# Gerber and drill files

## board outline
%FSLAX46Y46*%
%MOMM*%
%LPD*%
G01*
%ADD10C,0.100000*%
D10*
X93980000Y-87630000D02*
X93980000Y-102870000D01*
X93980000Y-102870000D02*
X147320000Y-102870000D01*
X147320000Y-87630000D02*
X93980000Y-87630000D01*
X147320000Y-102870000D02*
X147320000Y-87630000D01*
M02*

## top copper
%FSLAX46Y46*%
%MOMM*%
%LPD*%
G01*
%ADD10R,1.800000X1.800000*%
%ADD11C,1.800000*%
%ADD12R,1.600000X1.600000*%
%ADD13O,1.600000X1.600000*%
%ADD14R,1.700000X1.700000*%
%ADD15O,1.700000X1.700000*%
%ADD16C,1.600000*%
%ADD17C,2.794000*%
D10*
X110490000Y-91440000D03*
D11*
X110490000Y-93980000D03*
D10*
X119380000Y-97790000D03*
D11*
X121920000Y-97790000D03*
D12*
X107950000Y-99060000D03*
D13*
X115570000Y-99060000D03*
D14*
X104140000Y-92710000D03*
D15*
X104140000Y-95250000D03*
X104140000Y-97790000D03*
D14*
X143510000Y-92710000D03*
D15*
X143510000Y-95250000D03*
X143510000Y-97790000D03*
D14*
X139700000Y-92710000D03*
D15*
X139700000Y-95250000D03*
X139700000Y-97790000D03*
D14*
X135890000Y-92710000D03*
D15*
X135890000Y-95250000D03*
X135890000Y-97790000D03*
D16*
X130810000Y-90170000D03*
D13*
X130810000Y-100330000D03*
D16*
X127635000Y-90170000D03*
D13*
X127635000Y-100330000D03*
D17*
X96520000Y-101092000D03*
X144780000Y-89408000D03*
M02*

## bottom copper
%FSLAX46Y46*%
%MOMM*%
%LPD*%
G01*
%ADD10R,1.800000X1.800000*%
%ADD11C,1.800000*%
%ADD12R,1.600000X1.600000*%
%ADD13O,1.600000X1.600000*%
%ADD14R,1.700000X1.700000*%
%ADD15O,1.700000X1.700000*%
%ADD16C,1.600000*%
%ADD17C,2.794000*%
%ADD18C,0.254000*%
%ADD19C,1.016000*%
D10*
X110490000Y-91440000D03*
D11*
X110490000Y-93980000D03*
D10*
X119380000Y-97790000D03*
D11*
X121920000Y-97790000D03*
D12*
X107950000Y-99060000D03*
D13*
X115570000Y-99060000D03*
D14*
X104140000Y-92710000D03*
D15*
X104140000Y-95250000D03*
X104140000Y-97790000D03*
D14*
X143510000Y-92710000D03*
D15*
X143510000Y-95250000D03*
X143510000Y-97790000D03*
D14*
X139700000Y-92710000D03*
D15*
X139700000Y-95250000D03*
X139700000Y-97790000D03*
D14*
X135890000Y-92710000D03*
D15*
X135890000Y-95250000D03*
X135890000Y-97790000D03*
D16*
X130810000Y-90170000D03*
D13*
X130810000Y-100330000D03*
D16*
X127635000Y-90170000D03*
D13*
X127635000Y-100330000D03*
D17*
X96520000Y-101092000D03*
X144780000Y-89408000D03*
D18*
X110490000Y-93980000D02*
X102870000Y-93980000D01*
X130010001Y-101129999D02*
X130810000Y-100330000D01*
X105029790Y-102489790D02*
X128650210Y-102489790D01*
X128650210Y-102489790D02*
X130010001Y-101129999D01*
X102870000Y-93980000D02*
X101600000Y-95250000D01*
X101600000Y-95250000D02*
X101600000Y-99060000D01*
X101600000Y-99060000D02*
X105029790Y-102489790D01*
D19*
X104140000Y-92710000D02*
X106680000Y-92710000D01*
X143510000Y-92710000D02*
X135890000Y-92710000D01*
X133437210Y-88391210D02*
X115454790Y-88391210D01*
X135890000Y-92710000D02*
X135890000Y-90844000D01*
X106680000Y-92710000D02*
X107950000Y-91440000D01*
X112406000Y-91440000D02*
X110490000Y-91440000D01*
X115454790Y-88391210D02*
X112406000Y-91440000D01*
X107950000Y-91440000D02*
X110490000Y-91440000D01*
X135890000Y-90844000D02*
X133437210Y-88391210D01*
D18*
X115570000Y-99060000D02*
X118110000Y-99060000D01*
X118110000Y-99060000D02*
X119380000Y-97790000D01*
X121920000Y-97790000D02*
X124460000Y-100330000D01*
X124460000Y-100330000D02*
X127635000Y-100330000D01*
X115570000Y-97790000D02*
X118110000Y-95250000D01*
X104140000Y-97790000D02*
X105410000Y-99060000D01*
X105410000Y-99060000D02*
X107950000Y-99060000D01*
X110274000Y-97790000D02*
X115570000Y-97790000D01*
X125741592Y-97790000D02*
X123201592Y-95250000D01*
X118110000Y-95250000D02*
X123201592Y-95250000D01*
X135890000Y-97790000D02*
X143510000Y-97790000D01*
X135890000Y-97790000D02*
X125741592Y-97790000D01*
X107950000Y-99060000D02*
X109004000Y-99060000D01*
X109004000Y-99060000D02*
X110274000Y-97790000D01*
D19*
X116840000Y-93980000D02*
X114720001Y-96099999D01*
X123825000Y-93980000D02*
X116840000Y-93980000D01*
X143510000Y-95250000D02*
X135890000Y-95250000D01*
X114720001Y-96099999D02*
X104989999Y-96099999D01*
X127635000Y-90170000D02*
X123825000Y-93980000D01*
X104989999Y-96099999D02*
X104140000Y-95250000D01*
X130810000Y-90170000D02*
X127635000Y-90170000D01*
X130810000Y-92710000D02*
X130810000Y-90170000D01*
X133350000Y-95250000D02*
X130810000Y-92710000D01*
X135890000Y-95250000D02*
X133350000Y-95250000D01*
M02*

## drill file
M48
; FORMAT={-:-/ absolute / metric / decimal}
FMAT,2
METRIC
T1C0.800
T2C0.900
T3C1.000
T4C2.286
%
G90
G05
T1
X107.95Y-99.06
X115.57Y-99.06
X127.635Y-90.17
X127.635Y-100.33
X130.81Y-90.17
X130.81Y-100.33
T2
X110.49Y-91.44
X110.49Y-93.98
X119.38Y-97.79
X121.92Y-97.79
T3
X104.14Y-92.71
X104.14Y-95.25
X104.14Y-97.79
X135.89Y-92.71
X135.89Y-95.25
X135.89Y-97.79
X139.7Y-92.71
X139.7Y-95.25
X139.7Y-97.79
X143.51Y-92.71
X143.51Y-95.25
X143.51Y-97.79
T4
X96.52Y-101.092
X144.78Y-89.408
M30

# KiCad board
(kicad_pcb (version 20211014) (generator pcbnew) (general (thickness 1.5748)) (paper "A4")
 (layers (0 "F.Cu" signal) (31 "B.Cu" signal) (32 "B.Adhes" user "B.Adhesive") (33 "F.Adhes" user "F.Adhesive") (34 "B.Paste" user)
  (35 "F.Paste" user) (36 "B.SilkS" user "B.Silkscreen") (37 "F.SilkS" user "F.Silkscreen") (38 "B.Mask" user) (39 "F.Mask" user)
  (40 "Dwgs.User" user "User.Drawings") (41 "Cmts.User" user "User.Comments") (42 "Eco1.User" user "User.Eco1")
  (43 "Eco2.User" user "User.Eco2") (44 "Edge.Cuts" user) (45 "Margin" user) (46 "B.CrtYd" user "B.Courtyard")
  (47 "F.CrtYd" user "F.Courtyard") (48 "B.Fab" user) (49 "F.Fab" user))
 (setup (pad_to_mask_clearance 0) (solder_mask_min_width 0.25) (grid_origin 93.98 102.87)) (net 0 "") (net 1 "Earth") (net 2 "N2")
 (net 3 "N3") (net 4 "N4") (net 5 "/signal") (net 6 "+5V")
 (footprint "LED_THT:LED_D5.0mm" (layer "F.Cu") (at 110.49 91.44 -90)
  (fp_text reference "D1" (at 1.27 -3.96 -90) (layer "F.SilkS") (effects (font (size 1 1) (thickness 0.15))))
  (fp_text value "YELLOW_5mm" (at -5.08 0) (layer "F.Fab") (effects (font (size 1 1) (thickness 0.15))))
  (pad "1" thru_hole rect locked (at 0 0 270) (size 1.8 1.8) (drill 0.9) (layers *.Cu *.Mask) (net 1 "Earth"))
  (pad "2" thru_hole circle locked (at 2.54 0 270) (size 1.8 1.8) (drill 0.9) (layers *.Cu *.Mask) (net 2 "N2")))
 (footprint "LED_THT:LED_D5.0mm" (layer "F.Cu") (at 119.38 97.79)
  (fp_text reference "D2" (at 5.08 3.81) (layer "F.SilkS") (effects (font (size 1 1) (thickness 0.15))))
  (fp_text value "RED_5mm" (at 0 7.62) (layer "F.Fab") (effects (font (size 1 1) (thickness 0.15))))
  (pad "1" thru_hole rect locked (at 0 0) (size 1.8 1.8) (drill 0.9) (layers *.Cu *.Mask) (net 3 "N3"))
  (pad "2" thru_hole circle locked (at 2.54 0) (size 1.8 1.8) (drill 0.9) (layers *.Cu *.Mask) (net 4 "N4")))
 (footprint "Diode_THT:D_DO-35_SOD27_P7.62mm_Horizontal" (layer "F.Cu") (at 107.95 99.06)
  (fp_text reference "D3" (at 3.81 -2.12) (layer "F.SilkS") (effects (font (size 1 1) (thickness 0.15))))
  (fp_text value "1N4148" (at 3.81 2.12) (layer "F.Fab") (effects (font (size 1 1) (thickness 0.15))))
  (pad "1" thru_hole rect locked (at 0 0) (size 1.6 1.6) (drill 0.8) (layers *.Cu *.Mask) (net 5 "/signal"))
  (pad "2" thru_hole oval locked (at 7.62 0) (size 1.6 1.6) (drill 0.8) (layers *.Cu *.Mask) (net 3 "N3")))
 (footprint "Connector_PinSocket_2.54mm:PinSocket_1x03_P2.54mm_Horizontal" (layer "F.Cu") (at 104.14 92.71)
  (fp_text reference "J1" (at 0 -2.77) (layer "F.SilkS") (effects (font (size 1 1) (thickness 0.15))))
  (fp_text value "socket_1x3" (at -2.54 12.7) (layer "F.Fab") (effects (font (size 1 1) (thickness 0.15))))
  (pad "1" thru_hole rect locked (at 0 0) (size 1.7 1.7) (drill 1) (layers *.Cu *.Mask) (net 1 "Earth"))
  (pad "2" thru_hole oval locked (at 0 2.54) (size 1.7 1.7) (drill 1) (layers *.Cu *.Mask) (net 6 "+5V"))
  (pad "3" thru_hole oval locked (at 0 5.08) (size 1.7 1.7) (drill 1) (layers *.Cu *.Mask) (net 5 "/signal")))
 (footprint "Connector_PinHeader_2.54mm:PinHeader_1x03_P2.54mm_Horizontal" (layer "F.Cu") (at 143.51 92.71)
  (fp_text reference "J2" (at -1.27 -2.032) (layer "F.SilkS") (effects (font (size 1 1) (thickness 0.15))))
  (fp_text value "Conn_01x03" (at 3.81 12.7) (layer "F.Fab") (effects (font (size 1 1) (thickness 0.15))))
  (pad "1" thru_hole rect locked (at 0 0) (size 1.7 1.7) (drill 1) (layers *.Cu *.Mask) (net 1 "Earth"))
  (pad "2" thru_hole oval locked (at 0 2.54) (size 1.7 1.7) (drill 1) (layers *.Cu *.Mask) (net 6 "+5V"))
  (pad "3" thru_hole oval locked (at 0 5.08) (size 1.7 1.7) (drill 1) (layers *.Cu *.Mask) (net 5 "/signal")))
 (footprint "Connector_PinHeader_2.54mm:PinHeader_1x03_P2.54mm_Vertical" (layer "F.Cu") (at 139.7 92.71)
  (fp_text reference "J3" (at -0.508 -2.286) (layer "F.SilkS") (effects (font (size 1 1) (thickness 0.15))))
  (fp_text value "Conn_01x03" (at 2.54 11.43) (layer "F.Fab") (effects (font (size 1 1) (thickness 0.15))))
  (pad "1" thru_hole rect locked (at 0 0) (size 1.7 1.7) (drill 1) (layers *.Cu *.Mask) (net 1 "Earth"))
  (pad "2" thru_hole oval locked (at 0 2.54) (size 1.7 1.7) (drill 1) (layers *.Cu *.Mask) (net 6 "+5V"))
  (pad "3" thru_hole oval locked (at 0 5.08) (size 1.7 1.7) (drill 1) (layers *.Cu *.Mask) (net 5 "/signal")))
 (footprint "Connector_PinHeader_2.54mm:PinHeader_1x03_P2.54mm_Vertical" (layer "F.Cu") (at 135.89 92.71)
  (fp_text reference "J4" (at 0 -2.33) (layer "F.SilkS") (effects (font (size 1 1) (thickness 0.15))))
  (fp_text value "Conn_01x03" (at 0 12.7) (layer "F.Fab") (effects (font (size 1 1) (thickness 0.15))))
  (pad "1" thru_hole rect locked (at 0 0) (size 1.7 1.7) (drill 1) (layers *.Cu *.Mask) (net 1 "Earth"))
  (pad "2" thru_hole oval locked (at 0 2.54) (size 1.7 1.7) (drill 1) (layers *.Cu *.Mask) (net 6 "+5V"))
  (pad "3" thru_hole oval locked (at 0 5.08) (size 1.7 1.7) (drill 1) (layers *.Cu *.Mask) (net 5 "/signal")))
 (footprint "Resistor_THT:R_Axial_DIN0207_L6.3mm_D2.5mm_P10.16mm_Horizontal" (layer "F.Cu") (at 130.81 90.17 -90)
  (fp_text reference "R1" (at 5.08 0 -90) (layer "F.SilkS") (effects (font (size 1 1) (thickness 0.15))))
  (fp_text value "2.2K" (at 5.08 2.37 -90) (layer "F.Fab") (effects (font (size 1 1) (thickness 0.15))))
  (pad "1" thru_hole circle locked (at 0 0 270) (size 1.6 1.6) (drill 0.8) (layers *.Cu *.Mask) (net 6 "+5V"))
  (pad "2" thru_hole oval locked (at 10.16 0 270) (size 1.6 1.6) (drill 0.8) (layers *.Cu *.Mask) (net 2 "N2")))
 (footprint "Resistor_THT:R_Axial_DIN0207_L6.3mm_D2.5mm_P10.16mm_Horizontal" (layer "F.Cu") (at 127.635 90.17 -90)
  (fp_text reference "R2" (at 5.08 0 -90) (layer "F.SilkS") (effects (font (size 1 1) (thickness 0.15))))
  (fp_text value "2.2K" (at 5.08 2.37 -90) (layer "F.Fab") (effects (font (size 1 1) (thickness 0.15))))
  (pad "1" thru_hole circle locked (at 0 0 270) (size 1.6 1.6) (drill 0.8) (layers *.Cu *.Mask) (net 6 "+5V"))
  (pad "2" thru_hole oval locked (at 10.16 0 270) (size 1.6 1.6) (drill 0.8) (layers *.Cu *.Mask) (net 4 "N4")))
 (gr_line (start 93.98 87.63) (end 93.98 102.87) (layer "Edge.Cuts") (width 0.1))
 (gr_line (start 93.98 102.87) (end 147.32 102.87) (layer "Edge.Cuts") (width 0.1))
 (gr_line (start 147.32 87.63) (end 93.98 87.63) (layer "Edge.Cuts") (width 0.1))
 (gr_line (start 147.32 102.87) (end 147.32 87.63) (layer "Edge.Cuts") (width 0.1))
 (via (at 96.52 101.092) (size 2.794) (drill 2.286) (layers "F.Cu" "B.Cu") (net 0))
 (via (at 144.78 89.408) (size 2.794) (drill 2.286) (layers "F.Cu" "B.Cu") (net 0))
 (segment (start 110.49 93.98) (end 102.87 93.98) (width 0.254) (layer "B.Cu") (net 2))
 (segment (start 130.010001 101.129999) (end 130.81 100.33) (width 0.254) (layer "B.Cu") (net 2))
 (segment (start 105.02979 102.48979) (end 128.65021 102.48979) (width 0.254) (layer "B.Cu") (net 2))
 (segment (start 128.65021 102.48979) (end 130.010001 101.129999) (width 0.254) (layer "B.Cu") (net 2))
 (segment (start 102.87 93.98) (end 101.6 95.25) (width 0.254) (layer "B.Cu") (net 2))
 (segment (start 101.6 95.25) (end 101.6 99.06) (width 0.254) (layer "B.Cu") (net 2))
 (segment (start 101.6 99.06) (end 105.02979 102.48979) (width 0.254) (layer "B.Cu") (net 2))
 (segment (start 104.14 92.71) (end 106.68 92.71) (width 1.016) (layer "B.Cu") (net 1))
 (segment (start 143.51 92.71) (end 135.89 92.71) (width 1.016) (layer "B.Cu") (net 1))
 (segment (start 133.43721 88.39121) (end 115.45479 88.39121) (width 1.016) (layer "B.Cu") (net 1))
 (segment (start 135.89 92.71) (end 135.89 90.844) (width 1.016) (layer "B.Cu") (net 1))
 (segment (start 106.68 92.71) (end 107.95 91.44) (width 1.016) (layer "B.Cu") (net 1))
 (segment (start 112.406 91.44) (end 110.49 91.44) (width 1.016) (layer "B.Cu") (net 1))
 (segment (start 115.45479 88.39121) (end 112.406 91.44) (width 1.016) (layer "B.Cu") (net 1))
 (segment (start 107.95 91.44) (end 110.49 91.44) (width 1.016) (layer "B.Cu") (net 1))
 (segment (start 135.89 90.844) (end 133.43721 88.39121) (width 1.016) (layer "B.Cu") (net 1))
 (segment (start 115.57 99.06) (end 118.11 99.06) (width 0.254) (layer "B.Cu") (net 3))
 (segment (start 118.11 99.06) (end 119.38 97.79) (width 0.254) (layer "B.Cu") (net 3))
 (segment (start 121.92 97.79) (end 124.46 100.33) (width 0.254) (layer "B.Cu") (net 4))
 (segment (start 124.46 100.33) (end 127.635 100.33) (width 0.254) (layer "B.Cu") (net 4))
 (segment (start 115.57 97.79) (end 118.11 95.25) (width 0.254) (layer "B.Cu") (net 5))
 (segment (start 104.14 97.79) (end 105.41 99.06) (width 0.254) (layer "B.Cu") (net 5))
 (segment (start 105.41 99.06) (end 107.95 99.06) (width 0.254) (layer "B.Cu") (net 5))
 (segment (start 110.274 97.79) (end 115.57 97.79) (width 0.254) (layer "B.Cu") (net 5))
 (segment (start 125.741592 97.79) (end 123.201592 95.25) (width 0.254) (layer "B.Cu") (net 5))
 (segment (start 118.11 95.25) (end 123.201592 95.25) (width 0.254) (layer "B.Cu") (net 5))
 (segment (start 135.89 97.79) (end 143.51 97.79) (width 0.254) (layer "B.Cu") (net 5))
 (segment (start 135.89 97.79) (end 125.741592 97.79) (width 0.254) (layer "B.Cu") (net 5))
 (segment (start 107.95 99.06) (end 109.004 99.06) (width 0.254) (layer "B.Cu") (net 5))
 (segment (start 109.004 99.06) (end 110.274 97.79) (width 0.254) (layer "B.Cu") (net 5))
 (segment (start 116.84 93.98) (end 114.720001 96.099999) (width 1.016) (layer "B.Cu") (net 6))
 (segment (start 123.825 93.98) (end 116.84 93.98) (width 1.016) (layer "B.Cu") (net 6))
 (segment (start 143.51 95.25) (end 135.89 95.25) (width 1.016) (layer "B.Cu") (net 6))
 (segment (start 114.720001 96.099999) (end 104.989999 96.099999) (width 1.016) (layer "B.Cu") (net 6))
 (segment (start 127.635 90.17) (end 123.825 93.98) (width 1.016) (layer "B.Cu") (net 6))
 (segment (start 104.989999 96.099999) (end 104.14 95.25) (width 1.016) (layer "B.Cu") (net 6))
 (segment (start 130.81 90.17) (end 127.635 90.17) (width 1.016) (layer "B.Cu") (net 6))
 (segment (start 130.81 92.71) (end 130.81 90.17) (width 1.016) (layer "B.Cu") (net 6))
 (segment (start 133.35 95.25) (end 130.81 92.71) (width 1.016) (layer "B.Cu") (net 6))
 (segment (start 135.89 95.25) (end 133.35 95.25) (width 1.016) (layer "B.Cu") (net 6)))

